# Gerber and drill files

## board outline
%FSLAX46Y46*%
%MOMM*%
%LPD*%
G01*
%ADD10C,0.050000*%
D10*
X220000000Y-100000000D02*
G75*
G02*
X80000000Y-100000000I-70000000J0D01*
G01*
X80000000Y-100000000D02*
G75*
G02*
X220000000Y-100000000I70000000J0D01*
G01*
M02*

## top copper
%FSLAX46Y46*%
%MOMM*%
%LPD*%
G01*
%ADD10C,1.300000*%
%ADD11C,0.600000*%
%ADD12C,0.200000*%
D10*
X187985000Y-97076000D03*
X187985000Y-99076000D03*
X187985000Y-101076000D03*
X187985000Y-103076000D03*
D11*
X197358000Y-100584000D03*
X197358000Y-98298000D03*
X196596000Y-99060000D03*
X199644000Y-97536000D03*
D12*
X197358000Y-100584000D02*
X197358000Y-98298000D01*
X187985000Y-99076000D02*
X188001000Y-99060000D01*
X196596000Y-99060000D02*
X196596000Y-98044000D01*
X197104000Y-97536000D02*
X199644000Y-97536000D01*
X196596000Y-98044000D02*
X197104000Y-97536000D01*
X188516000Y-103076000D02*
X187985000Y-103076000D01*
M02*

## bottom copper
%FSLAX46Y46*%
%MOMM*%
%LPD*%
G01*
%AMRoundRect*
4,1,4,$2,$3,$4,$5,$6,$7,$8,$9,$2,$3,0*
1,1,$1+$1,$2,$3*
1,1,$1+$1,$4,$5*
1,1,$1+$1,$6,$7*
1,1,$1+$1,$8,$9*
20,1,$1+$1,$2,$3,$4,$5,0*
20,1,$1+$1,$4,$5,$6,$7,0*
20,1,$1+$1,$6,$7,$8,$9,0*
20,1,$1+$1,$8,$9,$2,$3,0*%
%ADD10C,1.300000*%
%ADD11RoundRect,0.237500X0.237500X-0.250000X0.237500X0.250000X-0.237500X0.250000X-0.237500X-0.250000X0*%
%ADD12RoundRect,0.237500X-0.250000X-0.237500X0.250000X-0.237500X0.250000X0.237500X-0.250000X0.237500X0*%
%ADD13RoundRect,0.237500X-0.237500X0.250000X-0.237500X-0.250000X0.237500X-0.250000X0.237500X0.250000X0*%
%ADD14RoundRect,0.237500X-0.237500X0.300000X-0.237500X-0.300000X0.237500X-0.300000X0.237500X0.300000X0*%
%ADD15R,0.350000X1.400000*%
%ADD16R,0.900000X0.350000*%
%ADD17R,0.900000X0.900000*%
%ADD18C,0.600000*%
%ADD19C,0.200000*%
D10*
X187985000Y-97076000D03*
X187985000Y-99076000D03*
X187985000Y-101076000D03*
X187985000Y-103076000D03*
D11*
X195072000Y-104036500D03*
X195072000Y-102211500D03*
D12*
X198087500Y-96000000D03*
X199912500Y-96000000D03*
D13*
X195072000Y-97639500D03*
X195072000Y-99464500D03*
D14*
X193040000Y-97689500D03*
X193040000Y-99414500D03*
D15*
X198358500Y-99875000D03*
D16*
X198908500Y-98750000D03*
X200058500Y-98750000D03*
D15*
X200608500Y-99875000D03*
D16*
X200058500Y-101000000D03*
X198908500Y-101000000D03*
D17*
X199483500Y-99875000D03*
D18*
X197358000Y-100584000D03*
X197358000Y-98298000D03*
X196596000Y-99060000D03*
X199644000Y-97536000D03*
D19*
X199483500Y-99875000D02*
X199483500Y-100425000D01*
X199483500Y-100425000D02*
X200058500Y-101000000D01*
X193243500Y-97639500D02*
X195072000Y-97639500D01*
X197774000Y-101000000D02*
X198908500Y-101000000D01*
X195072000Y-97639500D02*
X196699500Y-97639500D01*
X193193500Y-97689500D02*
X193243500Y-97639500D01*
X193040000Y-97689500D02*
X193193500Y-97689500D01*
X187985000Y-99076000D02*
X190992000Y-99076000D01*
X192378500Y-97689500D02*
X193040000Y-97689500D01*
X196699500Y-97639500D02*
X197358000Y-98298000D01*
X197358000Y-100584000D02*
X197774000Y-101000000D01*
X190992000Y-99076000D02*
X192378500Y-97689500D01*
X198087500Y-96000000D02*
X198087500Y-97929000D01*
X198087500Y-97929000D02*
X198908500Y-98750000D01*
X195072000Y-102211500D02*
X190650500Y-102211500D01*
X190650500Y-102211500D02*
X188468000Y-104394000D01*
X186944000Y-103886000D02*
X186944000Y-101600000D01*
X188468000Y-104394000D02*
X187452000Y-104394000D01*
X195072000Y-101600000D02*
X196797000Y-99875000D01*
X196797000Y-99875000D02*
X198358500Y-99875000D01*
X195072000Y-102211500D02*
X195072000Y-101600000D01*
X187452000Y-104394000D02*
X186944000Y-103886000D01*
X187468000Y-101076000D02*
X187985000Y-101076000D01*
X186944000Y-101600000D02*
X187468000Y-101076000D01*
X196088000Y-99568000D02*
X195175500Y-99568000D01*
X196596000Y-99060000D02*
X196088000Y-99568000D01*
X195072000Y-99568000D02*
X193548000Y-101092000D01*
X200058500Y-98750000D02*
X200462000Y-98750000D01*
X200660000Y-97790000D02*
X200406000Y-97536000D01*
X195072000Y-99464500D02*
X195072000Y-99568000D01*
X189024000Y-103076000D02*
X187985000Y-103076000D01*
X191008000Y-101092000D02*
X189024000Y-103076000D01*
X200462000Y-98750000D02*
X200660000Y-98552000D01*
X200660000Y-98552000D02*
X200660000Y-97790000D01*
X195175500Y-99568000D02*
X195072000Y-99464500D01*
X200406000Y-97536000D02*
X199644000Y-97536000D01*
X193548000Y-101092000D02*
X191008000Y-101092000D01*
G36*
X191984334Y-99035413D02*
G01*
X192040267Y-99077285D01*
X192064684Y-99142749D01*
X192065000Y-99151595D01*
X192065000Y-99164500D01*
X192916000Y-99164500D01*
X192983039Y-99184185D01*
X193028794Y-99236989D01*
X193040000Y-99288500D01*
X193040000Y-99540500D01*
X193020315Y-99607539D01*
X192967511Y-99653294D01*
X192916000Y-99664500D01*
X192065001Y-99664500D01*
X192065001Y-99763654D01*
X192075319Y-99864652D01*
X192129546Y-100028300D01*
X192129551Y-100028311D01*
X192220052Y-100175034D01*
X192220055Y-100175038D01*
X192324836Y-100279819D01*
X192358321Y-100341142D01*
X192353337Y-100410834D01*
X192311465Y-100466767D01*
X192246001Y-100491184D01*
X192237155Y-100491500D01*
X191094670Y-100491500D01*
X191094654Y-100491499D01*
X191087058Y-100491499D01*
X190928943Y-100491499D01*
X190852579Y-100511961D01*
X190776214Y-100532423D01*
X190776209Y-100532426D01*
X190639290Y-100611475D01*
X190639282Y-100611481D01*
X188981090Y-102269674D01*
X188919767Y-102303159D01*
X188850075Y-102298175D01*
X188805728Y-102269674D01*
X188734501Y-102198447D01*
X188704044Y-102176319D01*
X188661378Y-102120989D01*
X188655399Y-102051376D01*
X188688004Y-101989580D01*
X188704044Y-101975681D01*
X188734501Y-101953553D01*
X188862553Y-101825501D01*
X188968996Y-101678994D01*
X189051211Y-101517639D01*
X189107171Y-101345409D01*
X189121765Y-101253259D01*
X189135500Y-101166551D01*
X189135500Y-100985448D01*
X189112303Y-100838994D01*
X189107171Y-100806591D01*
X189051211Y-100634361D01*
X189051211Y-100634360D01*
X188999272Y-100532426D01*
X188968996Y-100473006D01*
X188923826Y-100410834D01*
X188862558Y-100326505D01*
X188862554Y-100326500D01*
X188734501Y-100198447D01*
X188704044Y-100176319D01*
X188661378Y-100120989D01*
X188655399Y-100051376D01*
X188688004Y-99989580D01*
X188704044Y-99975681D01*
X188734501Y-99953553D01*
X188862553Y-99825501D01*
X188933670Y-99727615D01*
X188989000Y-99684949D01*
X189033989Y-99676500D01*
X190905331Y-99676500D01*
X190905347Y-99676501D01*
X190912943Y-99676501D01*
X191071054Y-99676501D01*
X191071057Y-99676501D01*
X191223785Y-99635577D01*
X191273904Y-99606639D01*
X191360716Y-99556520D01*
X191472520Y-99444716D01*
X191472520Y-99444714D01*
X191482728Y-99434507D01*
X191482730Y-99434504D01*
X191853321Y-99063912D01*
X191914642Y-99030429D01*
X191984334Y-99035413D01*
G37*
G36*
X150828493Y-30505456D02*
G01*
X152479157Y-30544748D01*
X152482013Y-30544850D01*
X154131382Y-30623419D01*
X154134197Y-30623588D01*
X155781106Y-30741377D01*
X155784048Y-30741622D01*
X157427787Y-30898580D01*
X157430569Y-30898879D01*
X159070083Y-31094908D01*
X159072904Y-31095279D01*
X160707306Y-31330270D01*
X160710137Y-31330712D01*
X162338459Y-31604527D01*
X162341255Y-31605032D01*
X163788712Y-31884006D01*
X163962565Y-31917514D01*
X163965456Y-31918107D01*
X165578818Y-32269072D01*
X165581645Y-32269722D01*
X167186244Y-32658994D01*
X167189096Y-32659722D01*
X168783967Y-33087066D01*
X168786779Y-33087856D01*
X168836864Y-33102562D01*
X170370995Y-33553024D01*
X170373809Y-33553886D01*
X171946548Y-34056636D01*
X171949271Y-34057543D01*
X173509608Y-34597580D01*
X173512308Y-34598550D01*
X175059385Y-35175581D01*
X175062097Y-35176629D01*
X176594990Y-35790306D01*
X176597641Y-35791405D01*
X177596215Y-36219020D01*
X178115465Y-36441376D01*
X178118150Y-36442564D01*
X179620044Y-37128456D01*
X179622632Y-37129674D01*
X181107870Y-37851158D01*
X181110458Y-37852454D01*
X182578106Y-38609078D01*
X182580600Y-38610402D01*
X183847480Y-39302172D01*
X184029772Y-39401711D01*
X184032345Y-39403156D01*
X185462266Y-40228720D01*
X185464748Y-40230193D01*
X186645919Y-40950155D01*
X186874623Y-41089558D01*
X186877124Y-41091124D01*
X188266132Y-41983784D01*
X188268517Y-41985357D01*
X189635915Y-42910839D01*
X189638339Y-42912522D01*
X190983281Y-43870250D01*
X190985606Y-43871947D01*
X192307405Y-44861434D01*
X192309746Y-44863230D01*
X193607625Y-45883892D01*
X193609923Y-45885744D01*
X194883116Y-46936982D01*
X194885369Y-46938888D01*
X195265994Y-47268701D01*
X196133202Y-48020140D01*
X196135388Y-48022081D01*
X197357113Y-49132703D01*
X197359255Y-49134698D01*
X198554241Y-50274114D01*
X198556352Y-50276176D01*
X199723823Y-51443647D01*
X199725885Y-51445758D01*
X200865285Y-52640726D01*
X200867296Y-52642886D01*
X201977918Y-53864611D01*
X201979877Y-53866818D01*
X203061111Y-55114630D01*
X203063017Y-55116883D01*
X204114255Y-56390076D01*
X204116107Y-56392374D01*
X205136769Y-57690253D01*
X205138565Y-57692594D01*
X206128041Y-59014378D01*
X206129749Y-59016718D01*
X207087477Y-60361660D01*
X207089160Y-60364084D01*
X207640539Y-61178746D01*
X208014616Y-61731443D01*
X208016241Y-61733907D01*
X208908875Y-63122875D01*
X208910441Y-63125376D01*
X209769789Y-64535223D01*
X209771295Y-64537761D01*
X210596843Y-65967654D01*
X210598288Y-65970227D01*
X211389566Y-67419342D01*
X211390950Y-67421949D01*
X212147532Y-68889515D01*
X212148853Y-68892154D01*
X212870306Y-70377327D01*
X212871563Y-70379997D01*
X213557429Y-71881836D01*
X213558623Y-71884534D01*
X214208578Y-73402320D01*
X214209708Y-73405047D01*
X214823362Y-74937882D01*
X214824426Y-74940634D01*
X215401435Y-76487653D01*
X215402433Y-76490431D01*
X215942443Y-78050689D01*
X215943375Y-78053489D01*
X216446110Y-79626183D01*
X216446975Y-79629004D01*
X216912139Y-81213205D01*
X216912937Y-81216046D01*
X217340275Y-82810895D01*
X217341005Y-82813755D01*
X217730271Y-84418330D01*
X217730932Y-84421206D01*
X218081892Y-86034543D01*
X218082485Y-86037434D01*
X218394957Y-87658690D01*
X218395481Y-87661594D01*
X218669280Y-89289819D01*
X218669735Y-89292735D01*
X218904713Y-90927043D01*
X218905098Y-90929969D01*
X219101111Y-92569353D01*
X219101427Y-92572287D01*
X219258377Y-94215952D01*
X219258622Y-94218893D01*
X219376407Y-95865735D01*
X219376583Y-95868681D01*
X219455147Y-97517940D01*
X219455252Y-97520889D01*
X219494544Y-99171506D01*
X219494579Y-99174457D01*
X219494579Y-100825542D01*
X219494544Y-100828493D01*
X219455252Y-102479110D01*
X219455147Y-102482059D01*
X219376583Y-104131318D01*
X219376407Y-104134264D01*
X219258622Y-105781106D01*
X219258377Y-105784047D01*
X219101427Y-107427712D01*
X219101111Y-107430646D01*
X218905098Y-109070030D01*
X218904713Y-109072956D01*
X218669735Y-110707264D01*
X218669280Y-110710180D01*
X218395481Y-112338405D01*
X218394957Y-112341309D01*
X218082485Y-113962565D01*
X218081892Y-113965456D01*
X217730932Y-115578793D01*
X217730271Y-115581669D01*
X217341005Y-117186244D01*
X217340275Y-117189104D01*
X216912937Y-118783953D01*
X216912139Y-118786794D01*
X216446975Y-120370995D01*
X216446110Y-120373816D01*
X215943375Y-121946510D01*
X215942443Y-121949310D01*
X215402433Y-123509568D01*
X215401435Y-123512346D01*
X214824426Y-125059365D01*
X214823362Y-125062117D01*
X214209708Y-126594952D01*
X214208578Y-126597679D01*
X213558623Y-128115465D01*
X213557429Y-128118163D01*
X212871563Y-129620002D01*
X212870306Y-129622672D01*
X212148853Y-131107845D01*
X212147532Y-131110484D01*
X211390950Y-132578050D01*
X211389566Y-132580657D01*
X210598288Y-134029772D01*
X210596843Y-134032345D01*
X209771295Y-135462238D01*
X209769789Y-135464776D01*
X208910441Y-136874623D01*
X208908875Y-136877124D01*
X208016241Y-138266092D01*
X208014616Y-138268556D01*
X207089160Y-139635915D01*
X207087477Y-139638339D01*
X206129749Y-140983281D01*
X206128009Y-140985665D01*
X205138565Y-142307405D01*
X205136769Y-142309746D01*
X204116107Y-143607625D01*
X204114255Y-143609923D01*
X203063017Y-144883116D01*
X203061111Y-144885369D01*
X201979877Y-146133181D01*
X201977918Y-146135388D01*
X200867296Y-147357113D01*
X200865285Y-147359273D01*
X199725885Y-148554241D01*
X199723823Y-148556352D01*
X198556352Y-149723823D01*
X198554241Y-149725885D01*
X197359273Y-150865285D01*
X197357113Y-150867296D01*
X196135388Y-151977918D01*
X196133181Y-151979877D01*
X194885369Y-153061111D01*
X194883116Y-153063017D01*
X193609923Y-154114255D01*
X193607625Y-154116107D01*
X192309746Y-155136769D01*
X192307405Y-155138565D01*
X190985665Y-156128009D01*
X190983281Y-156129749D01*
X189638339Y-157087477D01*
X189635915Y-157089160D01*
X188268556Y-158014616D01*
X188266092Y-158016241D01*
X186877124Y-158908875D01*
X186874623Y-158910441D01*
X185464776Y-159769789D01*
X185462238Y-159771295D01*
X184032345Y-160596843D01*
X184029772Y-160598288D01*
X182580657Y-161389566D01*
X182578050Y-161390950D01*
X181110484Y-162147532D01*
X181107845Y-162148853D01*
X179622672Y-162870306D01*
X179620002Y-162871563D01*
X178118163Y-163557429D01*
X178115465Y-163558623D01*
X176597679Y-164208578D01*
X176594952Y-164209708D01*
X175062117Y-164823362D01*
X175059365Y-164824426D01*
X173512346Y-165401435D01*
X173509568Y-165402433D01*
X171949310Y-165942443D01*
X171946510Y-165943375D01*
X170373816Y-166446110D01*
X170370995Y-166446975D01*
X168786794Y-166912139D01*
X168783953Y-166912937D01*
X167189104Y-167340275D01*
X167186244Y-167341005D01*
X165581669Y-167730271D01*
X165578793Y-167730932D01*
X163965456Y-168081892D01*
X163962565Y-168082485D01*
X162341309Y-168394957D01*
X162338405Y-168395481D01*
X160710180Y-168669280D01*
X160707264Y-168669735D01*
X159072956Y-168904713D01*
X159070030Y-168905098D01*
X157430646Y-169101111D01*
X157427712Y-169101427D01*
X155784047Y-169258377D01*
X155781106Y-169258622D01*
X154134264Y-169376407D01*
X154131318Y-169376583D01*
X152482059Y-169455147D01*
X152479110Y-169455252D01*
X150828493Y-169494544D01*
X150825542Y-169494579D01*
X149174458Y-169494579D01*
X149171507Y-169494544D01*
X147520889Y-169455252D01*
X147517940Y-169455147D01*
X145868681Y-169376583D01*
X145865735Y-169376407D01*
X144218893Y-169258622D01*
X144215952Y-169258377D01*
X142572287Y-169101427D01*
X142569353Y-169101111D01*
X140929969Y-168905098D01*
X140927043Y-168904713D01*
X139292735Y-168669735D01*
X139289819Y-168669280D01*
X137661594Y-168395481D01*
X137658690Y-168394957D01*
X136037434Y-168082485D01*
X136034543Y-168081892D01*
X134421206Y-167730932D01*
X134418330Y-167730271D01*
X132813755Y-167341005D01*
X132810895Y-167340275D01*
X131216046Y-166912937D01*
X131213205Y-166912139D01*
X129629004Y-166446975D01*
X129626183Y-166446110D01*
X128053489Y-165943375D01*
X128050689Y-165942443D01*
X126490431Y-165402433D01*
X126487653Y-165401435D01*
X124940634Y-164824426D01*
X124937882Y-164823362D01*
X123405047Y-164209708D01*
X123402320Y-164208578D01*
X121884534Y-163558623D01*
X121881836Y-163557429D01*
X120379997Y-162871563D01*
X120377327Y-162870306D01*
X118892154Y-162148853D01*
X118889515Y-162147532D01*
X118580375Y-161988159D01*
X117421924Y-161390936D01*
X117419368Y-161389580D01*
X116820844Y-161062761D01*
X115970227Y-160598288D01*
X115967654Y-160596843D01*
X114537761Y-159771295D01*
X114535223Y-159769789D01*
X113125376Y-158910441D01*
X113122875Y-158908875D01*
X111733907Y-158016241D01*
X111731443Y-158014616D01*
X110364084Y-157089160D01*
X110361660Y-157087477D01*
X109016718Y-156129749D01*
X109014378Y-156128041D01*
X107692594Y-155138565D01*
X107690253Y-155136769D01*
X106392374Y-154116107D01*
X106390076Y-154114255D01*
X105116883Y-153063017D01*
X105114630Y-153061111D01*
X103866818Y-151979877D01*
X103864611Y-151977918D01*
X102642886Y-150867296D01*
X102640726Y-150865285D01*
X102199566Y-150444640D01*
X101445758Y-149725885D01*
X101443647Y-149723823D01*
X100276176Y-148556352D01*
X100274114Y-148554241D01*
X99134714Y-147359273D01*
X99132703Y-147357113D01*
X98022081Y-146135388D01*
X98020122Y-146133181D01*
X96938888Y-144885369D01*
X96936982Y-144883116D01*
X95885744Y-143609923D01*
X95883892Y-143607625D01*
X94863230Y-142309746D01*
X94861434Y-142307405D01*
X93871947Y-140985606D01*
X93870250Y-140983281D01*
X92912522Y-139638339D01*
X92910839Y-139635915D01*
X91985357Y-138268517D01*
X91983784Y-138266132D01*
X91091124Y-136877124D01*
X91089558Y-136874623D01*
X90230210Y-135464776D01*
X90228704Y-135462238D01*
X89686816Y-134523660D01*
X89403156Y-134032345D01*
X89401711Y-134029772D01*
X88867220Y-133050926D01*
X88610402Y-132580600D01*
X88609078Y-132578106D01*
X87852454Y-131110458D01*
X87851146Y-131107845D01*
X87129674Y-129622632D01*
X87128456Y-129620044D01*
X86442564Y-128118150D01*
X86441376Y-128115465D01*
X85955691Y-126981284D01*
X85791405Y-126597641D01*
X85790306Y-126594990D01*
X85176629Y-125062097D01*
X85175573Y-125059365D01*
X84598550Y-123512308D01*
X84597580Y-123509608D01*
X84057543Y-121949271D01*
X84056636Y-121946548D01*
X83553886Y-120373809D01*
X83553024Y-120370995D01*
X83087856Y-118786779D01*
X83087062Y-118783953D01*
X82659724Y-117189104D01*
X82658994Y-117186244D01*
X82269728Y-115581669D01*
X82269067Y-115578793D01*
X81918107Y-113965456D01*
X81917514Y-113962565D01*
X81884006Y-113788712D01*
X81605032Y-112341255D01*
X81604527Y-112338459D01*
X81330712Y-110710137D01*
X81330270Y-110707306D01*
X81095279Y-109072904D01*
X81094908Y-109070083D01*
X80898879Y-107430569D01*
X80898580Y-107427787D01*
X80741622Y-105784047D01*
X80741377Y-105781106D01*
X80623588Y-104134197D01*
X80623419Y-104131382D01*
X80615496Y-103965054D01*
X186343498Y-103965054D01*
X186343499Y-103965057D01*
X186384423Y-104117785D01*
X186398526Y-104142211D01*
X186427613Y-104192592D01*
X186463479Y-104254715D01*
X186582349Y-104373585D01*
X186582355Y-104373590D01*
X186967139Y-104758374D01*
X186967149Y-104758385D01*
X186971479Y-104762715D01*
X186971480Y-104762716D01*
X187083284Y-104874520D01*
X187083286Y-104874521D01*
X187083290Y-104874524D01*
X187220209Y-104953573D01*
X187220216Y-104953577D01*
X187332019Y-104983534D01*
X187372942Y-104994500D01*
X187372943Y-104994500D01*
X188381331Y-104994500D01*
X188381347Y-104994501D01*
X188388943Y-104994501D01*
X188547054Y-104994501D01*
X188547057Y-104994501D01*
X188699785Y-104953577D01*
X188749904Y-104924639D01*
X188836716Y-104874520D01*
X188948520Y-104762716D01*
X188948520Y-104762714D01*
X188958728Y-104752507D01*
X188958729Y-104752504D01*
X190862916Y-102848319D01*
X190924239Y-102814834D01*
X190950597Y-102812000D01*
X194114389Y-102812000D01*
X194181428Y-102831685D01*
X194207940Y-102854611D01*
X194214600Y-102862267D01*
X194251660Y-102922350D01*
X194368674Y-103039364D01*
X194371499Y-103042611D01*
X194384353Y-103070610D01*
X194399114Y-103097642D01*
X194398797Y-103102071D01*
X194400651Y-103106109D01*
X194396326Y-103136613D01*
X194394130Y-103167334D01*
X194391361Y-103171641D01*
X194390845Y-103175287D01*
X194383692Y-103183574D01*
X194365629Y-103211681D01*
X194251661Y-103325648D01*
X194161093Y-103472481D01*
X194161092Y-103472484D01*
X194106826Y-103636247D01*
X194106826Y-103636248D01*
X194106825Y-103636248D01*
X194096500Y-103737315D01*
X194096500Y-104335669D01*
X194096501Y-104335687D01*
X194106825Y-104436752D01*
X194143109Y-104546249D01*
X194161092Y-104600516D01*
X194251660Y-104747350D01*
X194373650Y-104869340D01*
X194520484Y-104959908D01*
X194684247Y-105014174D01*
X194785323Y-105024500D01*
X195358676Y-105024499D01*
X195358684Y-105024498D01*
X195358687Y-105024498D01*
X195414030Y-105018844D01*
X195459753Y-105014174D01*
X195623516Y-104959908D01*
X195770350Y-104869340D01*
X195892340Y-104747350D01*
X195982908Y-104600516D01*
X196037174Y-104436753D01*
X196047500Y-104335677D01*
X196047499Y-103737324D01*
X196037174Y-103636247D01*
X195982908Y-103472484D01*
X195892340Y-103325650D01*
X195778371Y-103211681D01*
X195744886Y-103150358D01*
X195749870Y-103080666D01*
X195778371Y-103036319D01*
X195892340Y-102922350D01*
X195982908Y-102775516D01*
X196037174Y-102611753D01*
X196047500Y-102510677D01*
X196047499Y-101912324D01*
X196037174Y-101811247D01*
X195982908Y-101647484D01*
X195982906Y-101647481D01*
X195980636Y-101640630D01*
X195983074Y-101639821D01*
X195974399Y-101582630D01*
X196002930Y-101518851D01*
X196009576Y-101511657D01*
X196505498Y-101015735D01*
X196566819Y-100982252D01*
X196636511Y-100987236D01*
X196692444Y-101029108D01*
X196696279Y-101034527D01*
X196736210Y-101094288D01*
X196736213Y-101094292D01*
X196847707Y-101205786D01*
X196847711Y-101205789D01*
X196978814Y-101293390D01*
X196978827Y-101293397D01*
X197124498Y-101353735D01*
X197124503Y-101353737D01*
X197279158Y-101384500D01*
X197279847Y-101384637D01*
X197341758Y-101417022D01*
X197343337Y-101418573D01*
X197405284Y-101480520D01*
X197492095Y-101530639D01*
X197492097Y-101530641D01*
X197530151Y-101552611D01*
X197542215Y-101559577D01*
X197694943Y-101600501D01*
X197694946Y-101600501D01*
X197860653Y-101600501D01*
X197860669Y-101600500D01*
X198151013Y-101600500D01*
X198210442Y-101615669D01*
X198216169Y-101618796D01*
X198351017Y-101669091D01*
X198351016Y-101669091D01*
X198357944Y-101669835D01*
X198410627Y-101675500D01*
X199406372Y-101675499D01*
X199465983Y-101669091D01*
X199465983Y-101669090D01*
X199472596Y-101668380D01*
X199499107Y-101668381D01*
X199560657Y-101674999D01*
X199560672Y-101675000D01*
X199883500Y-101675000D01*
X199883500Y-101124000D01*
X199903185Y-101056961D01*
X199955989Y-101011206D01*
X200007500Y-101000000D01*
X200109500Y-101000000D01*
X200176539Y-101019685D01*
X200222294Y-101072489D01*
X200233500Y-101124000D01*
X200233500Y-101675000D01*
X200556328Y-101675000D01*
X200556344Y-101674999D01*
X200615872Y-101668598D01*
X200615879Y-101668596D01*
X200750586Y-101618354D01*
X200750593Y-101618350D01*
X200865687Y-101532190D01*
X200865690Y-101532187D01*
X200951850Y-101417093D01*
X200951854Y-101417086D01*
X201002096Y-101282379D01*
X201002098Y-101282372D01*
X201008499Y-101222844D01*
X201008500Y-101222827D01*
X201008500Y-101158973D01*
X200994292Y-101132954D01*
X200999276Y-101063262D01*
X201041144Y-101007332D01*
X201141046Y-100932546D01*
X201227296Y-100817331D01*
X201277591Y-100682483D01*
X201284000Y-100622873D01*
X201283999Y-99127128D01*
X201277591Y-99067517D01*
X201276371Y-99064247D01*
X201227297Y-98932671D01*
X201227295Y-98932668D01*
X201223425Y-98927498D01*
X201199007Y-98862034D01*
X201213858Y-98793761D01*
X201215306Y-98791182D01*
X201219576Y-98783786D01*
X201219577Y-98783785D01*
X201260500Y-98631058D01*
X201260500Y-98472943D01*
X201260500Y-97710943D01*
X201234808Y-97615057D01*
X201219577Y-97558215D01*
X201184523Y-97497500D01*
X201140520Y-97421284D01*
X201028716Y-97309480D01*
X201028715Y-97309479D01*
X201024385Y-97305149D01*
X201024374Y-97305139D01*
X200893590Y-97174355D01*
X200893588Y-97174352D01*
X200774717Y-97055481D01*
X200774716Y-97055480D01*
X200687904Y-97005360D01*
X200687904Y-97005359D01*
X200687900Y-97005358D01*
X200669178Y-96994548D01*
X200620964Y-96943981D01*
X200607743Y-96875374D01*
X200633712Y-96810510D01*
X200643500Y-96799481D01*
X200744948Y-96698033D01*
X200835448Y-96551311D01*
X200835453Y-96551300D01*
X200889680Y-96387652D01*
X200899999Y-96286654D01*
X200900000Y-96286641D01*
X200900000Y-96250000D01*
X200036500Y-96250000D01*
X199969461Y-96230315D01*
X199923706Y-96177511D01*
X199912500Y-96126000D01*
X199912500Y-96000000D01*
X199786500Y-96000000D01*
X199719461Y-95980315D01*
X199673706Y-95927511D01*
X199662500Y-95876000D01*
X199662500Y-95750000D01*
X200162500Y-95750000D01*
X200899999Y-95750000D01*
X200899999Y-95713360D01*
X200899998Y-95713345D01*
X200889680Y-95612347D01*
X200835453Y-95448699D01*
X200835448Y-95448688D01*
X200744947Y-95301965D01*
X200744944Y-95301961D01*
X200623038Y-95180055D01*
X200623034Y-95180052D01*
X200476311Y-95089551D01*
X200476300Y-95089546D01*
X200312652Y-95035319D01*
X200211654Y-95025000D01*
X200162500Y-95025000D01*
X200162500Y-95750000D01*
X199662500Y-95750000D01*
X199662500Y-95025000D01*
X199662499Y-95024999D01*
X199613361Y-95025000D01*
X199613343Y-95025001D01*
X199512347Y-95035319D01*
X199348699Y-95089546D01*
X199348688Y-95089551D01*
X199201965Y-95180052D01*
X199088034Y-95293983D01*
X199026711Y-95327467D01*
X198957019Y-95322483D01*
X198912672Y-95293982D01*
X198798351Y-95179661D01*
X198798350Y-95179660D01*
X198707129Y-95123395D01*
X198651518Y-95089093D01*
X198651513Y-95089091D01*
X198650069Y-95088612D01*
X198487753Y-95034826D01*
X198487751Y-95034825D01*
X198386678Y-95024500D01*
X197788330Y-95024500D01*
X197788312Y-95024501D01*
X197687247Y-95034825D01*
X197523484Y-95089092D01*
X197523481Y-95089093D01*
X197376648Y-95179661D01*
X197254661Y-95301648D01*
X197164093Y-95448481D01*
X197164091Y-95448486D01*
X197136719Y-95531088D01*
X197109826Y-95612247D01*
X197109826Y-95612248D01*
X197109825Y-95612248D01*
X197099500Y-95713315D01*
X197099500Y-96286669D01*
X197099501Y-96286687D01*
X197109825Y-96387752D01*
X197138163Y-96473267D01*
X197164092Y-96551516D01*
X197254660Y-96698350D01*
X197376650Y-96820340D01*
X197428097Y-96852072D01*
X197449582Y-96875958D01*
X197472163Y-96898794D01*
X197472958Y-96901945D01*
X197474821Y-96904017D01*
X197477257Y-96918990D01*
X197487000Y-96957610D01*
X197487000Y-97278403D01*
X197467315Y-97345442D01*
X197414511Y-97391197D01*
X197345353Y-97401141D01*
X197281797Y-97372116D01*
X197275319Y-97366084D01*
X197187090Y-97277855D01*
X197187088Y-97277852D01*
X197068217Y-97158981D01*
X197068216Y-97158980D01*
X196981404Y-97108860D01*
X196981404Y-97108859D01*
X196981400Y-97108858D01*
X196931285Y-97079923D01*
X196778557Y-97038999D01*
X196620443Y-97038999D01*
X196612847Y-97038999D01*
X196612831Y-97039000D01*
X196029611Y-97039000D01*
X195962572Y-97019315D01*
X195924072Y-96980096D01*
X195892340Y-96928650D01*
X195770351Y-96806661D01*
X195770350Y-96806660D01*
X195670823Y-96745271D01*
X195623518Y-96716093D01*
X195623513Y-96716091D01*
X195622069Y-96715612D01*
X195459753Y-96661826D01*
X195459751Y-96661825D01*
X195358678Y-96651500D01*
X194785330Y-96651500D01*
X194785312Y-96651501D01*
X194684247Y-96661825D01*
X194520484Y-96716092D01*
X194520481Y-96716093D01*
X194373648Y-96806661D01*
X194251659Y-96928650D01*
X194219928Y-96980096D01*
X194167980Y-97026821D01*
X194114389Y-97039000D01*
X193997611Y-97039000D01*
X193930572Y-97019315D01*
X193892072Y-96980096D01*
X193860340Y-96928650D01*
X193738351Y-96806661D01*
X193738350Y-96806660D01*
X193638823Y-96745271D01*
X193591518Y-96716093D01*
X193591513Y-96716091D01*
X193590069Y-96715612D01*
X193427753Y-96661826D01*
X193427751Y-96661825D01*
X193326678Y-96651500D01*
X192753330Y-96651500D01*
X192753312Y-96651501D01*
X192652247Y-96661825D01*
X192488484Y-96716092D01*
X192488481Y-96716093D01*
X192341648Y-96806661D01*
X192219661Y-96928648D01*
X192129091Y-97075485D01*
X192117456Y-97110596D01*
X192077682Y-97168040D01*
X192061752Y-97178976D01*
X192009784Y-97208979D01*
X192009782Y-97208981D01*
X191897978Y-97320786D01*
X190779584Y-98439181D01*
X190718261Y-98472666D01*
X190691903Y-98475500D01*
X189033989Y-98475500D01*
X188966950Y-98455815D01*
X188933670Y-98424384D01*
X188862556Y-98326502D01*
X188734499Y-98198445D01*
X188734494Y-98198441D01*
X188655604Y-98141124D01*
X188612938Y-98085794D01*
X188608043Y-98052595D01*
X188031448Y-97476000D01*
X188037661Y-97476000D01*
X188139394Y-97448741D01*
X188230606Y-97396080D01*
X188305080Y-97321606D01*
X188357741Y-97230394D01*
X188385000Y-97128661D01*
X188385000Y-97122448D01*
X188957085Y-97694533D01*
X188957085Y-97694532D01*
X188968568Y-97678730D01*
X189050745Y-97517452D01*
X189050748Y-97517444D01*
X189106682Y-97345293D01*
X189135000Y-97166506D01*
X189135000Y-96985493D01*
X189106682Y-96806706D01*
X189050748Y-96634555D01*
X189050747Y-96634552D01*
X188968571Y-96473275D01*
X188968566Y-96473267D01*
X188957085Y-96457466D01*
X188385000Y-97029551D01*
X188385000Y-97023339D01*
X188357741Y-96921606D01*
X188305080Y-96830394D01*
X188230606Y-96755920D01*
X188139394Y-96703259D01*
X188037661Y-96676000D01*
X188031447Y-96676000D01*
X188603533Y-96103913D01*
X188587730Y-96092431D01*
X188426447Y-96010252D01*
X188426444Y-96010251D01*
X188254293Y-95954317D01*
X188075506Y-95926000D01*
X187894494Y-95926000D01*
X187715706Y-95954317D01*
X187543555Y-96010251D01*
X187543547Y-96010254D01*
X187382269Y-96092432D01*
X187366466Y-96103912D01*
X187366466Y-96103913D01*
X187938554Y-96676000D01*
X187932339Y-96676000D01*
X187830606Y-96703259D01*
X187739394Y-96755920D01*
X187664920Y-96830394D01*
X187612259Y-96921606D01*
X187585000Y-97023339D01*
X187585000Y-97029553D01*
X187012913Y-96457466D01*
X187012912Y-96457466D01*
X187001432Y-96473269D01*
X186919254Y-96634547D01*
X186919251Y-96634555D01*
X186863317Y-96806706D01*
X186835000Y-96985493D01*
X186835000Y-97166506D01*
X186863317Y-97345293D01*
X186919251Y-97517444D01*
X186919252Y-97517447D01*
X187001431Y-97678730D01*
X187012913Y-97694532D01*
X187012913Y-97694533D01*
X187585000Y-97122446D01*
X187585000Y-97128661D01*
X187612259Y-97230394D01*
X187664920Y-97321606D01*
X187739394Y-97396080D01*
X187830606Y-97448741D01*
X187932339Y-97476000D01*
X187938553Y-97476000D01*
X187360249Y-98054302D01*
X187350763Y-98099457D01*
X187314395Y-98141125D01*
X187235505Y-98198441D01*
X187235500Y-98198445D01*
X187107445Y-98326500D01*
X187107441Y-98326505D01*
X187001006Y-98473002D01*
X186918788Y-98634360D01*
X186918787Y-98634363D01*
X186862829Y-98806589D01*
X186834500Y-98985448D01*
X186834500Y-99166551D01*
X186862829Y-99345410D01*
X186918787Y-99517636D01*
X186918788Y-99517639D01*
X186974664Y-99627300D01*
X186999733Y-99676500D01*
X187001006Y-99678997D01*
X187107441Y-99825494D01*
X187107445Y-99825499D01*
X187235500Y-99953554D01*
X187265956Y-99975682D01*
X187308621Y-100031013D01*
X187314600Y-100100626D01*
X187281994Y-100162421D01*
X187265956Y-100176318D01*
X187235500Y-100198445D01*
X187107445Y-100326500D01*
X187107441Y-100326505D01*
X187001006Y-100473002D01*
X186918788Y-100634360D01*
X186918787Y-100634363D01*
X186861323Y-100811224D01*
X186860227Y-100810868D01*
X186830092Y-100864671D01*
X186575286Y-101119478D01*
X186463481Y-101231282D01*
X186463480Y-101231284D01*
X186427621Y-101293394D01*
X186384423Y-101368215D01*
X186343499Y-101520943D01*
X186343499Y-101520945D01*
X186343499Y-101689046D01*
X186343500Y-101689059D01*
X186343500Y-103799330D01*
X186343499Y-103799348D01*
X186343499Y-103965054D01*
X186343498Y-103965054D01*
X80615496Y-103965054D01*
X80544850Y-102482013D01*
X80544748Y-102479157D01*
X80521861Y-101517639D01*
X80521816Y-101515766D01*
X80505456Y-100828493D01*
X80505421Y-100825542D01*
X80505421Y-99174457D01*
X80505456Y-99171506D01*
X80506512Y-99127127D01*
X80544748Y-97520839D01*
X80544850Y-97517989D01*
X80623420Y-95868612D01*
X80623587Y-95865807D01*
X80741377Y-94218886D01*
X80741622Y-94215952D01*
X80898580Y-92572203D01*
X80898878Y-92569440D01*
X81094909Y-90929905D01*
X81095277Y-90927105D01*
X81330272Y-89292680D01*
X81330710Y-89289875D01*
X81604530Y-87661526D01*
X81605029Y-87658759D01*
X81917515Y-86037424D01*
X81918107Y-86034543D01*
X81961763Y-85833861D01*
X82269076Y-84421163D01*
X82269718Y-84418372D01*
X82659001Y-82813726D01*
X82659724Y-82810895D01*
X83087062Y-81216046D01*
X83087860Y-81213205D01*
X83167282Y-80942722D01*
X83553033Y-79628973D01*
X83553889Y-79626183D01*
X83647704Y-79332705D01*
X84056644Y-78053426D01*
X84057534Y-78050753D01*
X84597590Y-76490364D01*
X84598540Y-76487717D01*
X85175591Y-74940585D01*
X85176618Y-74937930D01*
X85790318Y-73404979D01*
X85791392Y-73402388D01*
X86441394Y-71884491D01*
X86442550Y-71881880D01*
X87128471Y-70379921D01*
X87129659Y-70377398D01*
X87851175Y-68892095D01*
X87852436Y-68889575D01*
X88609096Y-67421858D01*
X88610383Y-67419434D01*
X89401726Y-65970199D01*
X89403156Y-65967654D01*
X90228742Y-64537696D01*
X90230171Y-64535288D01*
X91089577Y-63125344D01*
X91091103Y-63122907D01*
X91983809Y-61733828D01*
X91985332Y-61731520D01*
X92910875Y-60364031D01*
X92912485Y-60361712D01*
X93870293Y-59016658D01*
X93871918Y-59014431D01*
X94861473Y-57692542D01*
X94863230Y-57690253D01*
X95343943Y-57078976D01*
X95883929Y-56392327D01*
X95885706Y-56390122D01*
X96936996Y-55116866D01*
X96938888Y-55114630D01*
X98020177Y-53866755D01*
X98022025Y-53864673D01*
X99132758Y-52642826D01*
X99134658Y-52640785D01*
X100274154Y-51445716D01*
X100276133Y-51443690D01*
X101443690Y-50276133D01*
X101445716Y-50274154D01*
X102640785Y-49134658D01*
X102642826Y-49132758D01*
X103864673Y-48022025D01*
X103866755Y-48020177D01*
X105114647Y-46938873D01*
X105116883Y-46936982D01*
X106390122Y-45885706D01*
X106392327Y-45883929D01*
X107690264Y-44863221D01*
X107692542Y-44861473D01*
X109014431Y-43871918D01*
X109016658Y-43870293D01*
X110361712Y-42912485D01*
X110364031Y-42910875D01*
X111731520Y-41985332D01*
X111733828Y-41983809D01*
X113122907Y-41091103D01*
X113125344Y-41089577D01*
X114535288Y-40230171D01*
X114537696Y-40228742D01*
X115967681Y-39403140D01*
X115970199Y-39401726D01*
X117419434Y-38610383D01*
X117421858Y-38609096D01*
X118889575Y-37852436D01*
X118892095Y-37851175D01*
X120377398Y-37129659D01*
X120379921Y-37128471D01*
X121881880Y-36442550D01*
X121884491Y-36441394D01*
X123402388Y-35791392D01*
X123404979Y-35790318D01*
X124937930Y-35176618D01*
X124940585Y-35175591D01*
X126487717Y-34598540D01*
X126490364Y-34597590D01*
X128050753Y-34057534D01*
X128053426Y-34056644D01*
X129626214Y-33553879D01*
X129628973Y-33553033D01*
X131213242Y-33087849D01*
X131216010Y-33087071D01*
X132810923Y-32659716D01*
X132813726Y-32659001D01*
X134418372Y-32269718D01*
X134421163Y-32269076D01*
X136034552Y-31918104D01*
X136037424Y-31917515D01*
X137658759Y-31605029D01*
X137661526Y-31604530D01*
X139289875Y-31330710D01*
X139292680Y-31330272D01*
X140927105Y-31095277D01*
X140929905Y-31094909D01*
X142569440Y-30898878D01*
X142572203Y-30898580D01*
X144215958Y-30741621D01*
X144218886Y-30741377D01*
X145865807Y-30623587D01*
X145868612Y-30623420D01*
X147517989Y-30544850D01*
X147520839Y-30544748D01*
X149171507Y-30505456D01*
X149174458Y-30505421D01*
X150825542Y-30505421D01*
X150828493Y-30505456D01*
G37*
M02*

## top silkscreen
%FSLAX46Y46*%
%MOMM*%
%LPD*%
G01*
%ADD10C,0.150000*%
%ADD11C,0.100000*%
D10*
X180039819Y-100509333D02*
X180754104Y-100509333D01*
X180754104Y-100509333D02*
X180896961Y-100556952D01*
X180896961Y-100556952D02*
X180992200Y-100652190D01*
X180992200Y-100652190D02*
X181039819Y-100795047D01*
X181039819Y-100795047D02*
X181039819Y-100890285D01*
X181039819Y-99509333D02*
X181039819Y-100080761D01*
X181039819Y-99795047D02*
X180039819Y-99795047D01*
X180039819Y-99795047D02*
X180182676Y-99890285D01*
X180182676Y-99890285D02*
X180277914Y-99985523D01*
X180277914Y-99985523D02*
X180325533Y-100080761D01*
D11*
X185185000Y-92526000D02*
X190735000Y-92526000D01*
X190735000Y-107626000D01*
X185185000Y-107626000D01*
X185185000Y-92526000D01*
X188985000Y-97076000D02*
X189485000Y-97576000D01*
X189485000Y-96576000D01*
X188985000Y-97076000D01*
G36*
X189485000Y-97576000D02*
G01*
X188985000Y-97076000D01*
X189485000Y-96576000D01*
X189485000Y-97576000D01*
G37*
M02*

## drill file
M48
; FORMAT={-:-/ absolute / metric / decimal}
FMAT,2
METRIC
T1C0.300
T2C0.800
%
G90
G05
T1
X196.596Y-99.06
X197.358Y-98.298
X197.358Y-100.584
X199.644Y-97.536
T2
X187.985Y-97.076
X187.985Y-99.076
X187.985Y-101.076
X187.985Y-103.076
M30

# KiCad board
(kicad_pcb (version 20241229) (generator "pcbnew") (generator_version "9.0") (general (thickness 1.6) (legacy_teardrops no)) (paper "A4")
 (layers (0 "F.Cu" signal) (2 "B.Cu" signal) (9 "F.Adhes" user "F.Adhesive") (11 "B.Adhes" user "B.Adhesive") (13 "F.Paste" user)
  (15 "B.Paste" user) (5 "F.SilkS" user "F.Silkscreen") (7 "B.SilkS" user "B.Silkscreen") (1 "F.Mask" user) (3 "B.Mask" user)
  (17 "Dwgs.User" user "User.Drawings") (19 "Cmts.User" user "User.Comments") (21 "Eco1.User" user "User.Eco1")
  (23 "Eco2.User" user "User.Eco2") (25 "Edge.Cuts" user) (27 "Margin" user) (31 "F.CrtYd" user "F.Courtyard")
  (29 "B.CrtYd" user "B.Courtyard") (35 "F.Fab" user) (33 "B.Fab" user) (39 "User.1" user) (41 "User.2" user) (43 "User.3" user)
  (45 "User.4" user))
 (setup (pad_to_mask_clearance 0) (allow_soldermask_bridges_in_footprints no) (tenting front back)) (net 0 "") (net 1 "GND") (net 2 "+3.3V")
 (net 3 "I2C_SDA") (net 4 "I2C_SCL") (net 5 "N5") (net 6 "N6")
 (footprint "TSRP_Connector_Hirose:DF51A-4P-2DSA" (layer "F.Cu") (at 190.585 100.076 90)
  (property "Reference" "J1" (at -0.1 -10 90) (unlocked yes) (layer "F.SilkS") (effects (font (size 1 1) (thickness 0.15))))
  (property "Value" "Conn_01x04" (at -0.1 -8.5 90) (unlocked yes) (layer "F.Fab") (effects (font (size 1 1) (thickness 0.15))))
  (fp_rect (start -7.55 -5.4) (end 7.55 0.15) (stroke (width 0.1) (type default)) (fill no) (layer "F.SilkS"))
  (fp_poly (pts (xy 3 -1.6) (xy 2.5 -1.1) (xy 3.5 -1.1)) (stroke (width 0.1) (type solid)) (fill yes) (layer "F.SilkS"))
  (pad "1" thru_hole circle (at 3 -2.6 90) (size 1.3 1.3) (drill 0.8) (layers "*.Cu" "*.Mask") (remove_unused_layers no) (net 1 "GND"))
  (pad "2" thru_hole circle (at 1 -2.6 90) (size 1.3 1.3) (drill 0.8) (layers "*.Cu" "*.Mask") (remove_unused_layers no) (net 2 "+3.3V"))
  (pad "3" thru_hole circle (at -1 -2.6 90) (size 1.3 1.3) (drill 0.8) (layers "*.Cu" "*.Mask") (remove_unused_layers no) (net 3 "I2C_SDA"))
  (pad "4" thru_hole circle (at -3 -2.6 90) (size 1.3 1.3) (drill 0.8) (layers "*.Cu" "*.Mask") (remove_unused_layers no) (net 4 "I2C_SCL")))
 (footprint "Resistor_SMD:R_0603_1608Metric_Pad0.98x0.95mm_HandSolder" (layer "B.Cu") (at 195.072 103.124 90)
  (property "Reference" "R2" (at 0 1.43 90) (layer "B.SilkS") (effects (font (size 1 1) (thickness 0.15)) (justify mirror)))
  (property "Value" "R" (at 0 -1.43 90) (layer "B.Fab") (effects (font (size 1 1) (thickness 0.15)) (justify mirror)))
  (pad "1" smd roundrect (at -0.9125 0 90) (size 0.975 0.95) (layers "B.Cu" "B.Mask" "B.Paste") (roundrect_rratio 0.25) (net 2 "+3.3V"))
  (pad "2" smd roundrect (at 0.9125 0 90) (size 0.975 0.95) (layers "B.Cu" "B.Mask" "B.Paste") (roundrect_rratio 0.25) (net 3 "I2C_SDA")))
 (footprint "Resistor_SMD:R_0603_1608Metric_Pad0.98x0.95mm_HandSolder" (layer "B.Cu") (at 199 96)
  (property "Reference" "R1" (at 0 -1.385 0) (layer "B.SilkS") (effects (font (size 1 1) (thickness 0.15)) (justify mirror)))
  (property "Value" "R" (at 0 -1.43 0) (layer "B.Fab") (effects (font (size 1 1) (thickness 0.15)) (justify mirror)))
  (pad "1" smd roundrect (at -0.9125 0) (size 0.975 0.95) (layers "B.Cu" "B.Mask" "B.Paste") (roundrect_rratio 0.25) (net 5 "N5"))
  (pad "2" smd roundrect (at 0.9125 0) (size 0.975 0.95) (layers "B.Cu" "B.Mask" "B.Paste") (roundrect_rratio 0.25) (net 1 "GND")))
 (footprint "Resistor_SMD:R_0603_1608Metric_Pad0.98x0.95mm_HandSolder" (layer "B.Cu") (at 195.072 98.552 -90)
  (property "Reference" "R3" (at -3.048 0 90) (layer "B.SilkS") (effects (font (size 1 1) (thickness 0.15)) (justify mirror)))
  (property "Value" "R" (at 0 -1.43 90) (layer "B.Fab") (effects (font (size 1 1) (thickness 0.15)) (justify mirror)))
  (pad "1" smd roundrect (at -0.9125 0 270) (size 0.975 0.95) (layers "B.Cu" "B.Mask" "B.Paste") (roundrect_rratio 0.25) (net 2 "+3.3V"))
  (pad "2" smd roundrect (at 0.9125 0 270) (size 0.975 0.95) (layers "B.Cu" "B.Mask" "B.Paste") (roundrect_rratio 0.25) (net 4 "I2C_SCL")))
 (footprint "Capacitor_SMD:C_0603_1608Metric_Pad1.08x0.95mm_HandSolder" (layer "B.Cu") (at 193.04 98.552 -90)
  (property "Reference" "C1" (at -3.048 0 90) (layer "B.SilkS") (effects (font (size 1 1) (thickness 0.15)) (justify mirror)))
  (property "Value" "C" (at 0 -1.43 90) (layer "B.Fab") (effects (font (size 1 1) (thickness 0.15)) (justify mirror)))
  (pad "1" smd roundrect (at -0.8625 0 270) (size 1.075 0.95) (layers "B.Cu" "B.Mask" "B.Paste") (roundrect_rratio 0.25) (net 2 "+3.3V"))
  (pad "2" smd roundrect (at 0.8625 0 270) (size 1.075 0.95) (layers "B.Cu" "B.Mask" "B.Paste") (roundrect_rratio 0.25) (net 1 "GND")))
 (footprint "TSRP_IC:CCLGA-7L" (layer "B.Cu") (at 199.4835 99.875 180)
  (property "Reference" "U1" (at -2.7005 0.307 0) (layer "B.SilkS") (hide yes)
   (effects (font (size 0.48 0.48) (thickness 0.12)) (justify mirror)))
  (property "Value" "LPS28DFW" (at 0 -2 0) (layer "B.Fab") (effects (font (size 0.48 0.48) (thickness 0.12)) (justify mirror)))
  (pad "1" smd rect (at 1.125 0 180) (size 0.35 1.4) (layers "B.Cu") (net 3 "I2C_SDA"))
  (pad "2" smd rect (at 0.575 1.125 180) (size 0.9 0.35) (layers "B.Cu") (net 5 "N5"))
  (pad "3" smd rect (at -0.575 1.125 180) (size 0.9 0.35) (layers "B.Cu") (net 4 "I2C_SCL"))
  (pad "4" smd rect (at -1.125 0 180) (size 0.35 1.4) (layers "B.Cu") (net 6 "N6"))
  (pad "5" smd rect (at -0.575 -1.125 180) (size 0.9 0.35) (layers "B.Cu") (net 1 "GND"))
  (pad "6" smd rect (at 0.575 -1.125 180) (size 0.9 0.35) (layers "B.Cu") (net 2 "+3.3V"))
  (pad "7" smd rect (at 0 0 180) (size 0.9 0.9) (layers "B.Cu") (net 1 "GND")))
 (gr_circle (center 150 100) (end 220 100) (stroke (width 0.05) (type default)) (fill no) (layer "Edge.Cuts"))
 (segment (start 199.4835 99.875) (end 199.4835 100.425) (width 0.2) (layer "B.Cu") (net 1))
 (segment (start 199.4835 100.425) (end 200.0585 101) (width 0.2) (layer "B.Cu") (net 1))
 (segment (start 197.358 100.584) (end 197.358 98.298) (width 0.2) (layer "F.Cu") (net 2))
 (segment (start 187.985 99.076) (end 188.001 99.06) (width 0.2) (layer "F.Cu") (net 2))
 (via (at 197.358 100.584) (size 0.6) (drill 0.3) (layers "F.Cu" "B.Cu") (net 2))
 (via (at 197.358 98.298) (size 0.6) (drill 0.3) (layers "F.Cu" "B.Cu") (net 2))
 (segment (start 193.2435 97.6395) (end 195.072 97.6395) (width 0.2) (layer "B.Cu") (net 2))
 (segment (start 197.774 101) (end 198.9085 101) (width 0.2) (layer "B.Cu") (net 2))
 (segment (start 195.072 97.6395) (end 196.6995 97.6395) (width 0.2) (layer "B.Cu") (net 2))
 (segment (start 193.1935 97.6895) (end 193.2435 97.6395) (width 0.2) (layer "B.Cu") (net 2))
 (segment (start 193.04 97.6895) (end 193.1935 97.6895) (width 0.2) (layer "B.Cu") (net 2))
 (segment (start 187.985 99.076) (end 190.992 99.076) (width 0.2) (layer "B.Cu") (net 2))
 (segment (start 192.3785 97.6895) (end 193.04 97.6895) (width 0.2) (layer "B.Cu") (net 2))
 (segment (start 196.6995 97.6395) (end 197.358 98.298) (width 0.2) (layer "B.Cu") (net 2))
 (segment (start 197.358 100.584) (end 197.774 101) (width 0.2) (layer "B.Cu") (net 2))
 (segment (start 190.992 99.076) (end 192.3785 97.6895) (width 0.2) (layer "B.Cu") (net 2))
 (segment (start 198.0875 96) (end 198.0875 97.929) (width 0.2) (layer "B.Cu") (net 5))
 (segment (start 198.0875 97.929) (end 198.9085 98.75) (width 0.2) (layer "B.Cu") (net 5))
 (segment (start 195.072 102.2115) (end 190.6505 102.2115) (width 0.2) (layer "B.Cu") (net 3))
 (segment (start 190.6505 102.2115) (end 188.468 104.394) (width 0.2) (layer "B.Cu") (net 3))
 (segment (start 186.944 103.886) (end 186.944 101.6) (width 0.2) (layer "B.Cu") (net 3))
 (segment (start 188.468 104.394) (end 187.452 104.394) (width 0.2) (layer "B.Cu") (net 3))
 (segment (start 195.072 101.6) (end 196.797 99.875) (width 0.2) (layer "B.Cu") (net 3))
 (segment (start 196.797 99.875) (end 198.3585 99.875) (width 0.2) (layer "B.Cu") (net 3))
 (segment (start 195.072 102.2115) (end 195.072 101.6) (width 0.2) (layer "B.Cu") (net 3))
 (segment (start 187.452 104.394) (end 186.944 103.886) (width 0.2) (layer "B.Cu") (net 3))
 (segment (start 187.468 101.076) (end 187.985 101.076) (width 0.2) (layer "B.Cu") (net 3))
 (segment (start 186.944 101.6) (end 187.468 101.076) (width 0.2) (layer "B.Cu") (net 3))
 (segment (start 196.596 99.06) (end 196.596 98.044) (width 0.2) (layer "F.Cu") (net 4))
 (segment (start 197.104 97.536) (end 199.644 97.536) (width 0.2) (layer "F.Cu") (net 4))
 (segment (start 196.596 98.044) (end 197.104 97.536) (width 0.2) (layer "F.Cu") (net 4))
 (segment (start 188.516 103.076) (end 187.985 103.076) (width 0.2) (layer "F.Cu") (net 4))
 (via (at 196.596 99.06) (size 0.6) (drill 0.3) (layers "F.Cu" "B.Cu") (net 4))
 (via (at 199.644 97.536) (size 0.6) (drill 0.3) (layers "F.Cu" "B.Cu") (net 4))
 (segment (start 196.088 99.568) (end 195.1755 99.568) (width 0.2) (layer "B.Cu") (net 4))
 (segment (start 196.596 99.06) (end 196.088 99.568) (width 0.2) (layer "B.Cu") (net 4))
 (segment (start 195.072 99.568) (end 193.548 101.092) (width 0.2) (layer "B.Cu") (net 4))
 (segment (start 200.0585 98.75) (end 200.462 98.75) (width 0.2) (layer "B.Cu") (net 4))
 (segment (start 200.66 97.79) (end 200.406 97.536) (width 0.2) (layer "B.Cu") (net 4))
 (segment (start 195.072 99.4645) (end 195.072 99.568) (width 0.2) (layer "B.Cu") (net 4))
 (segment (start 189.024 103.076) (end 187.985 103.076) (width 0.2) (layer "B.Cu") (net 4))
 (segment (start 191.008 101.092) (end 189.024 103.076) (width 0.2) (layer "B.Cu") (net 4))
 (segment (start 200.462 98.75) (end 200.66 98.552) (width 0.2) (layer "B.Cu") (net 4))
 (segment (start 200.66 98.552) (end 200.66 97.79) (width 0.2) (layer "B.Cu") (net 4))
 (segment (start 195.1755 99.568) (end 195.072 99.4645) (width 0.2) (layer "B.Cu") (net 4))
 (segment (start 200.406 97.536) (end 199.644 97.536) (width 0.2) (layer "B.Cu") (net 4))
 (segment (start 193.548 101.092) (end 191.008 101.092) (width 0.2) (layer "B.Cu") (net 4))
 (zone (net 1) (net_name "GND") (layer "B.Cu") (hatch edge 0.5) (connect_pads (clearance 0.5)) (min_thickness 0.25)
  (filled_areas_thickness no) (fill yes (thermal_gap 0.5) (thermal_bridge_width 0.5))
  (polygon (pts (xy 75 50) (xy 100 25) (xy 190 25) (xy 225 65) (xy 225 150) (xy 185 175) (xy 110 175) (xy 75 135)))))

